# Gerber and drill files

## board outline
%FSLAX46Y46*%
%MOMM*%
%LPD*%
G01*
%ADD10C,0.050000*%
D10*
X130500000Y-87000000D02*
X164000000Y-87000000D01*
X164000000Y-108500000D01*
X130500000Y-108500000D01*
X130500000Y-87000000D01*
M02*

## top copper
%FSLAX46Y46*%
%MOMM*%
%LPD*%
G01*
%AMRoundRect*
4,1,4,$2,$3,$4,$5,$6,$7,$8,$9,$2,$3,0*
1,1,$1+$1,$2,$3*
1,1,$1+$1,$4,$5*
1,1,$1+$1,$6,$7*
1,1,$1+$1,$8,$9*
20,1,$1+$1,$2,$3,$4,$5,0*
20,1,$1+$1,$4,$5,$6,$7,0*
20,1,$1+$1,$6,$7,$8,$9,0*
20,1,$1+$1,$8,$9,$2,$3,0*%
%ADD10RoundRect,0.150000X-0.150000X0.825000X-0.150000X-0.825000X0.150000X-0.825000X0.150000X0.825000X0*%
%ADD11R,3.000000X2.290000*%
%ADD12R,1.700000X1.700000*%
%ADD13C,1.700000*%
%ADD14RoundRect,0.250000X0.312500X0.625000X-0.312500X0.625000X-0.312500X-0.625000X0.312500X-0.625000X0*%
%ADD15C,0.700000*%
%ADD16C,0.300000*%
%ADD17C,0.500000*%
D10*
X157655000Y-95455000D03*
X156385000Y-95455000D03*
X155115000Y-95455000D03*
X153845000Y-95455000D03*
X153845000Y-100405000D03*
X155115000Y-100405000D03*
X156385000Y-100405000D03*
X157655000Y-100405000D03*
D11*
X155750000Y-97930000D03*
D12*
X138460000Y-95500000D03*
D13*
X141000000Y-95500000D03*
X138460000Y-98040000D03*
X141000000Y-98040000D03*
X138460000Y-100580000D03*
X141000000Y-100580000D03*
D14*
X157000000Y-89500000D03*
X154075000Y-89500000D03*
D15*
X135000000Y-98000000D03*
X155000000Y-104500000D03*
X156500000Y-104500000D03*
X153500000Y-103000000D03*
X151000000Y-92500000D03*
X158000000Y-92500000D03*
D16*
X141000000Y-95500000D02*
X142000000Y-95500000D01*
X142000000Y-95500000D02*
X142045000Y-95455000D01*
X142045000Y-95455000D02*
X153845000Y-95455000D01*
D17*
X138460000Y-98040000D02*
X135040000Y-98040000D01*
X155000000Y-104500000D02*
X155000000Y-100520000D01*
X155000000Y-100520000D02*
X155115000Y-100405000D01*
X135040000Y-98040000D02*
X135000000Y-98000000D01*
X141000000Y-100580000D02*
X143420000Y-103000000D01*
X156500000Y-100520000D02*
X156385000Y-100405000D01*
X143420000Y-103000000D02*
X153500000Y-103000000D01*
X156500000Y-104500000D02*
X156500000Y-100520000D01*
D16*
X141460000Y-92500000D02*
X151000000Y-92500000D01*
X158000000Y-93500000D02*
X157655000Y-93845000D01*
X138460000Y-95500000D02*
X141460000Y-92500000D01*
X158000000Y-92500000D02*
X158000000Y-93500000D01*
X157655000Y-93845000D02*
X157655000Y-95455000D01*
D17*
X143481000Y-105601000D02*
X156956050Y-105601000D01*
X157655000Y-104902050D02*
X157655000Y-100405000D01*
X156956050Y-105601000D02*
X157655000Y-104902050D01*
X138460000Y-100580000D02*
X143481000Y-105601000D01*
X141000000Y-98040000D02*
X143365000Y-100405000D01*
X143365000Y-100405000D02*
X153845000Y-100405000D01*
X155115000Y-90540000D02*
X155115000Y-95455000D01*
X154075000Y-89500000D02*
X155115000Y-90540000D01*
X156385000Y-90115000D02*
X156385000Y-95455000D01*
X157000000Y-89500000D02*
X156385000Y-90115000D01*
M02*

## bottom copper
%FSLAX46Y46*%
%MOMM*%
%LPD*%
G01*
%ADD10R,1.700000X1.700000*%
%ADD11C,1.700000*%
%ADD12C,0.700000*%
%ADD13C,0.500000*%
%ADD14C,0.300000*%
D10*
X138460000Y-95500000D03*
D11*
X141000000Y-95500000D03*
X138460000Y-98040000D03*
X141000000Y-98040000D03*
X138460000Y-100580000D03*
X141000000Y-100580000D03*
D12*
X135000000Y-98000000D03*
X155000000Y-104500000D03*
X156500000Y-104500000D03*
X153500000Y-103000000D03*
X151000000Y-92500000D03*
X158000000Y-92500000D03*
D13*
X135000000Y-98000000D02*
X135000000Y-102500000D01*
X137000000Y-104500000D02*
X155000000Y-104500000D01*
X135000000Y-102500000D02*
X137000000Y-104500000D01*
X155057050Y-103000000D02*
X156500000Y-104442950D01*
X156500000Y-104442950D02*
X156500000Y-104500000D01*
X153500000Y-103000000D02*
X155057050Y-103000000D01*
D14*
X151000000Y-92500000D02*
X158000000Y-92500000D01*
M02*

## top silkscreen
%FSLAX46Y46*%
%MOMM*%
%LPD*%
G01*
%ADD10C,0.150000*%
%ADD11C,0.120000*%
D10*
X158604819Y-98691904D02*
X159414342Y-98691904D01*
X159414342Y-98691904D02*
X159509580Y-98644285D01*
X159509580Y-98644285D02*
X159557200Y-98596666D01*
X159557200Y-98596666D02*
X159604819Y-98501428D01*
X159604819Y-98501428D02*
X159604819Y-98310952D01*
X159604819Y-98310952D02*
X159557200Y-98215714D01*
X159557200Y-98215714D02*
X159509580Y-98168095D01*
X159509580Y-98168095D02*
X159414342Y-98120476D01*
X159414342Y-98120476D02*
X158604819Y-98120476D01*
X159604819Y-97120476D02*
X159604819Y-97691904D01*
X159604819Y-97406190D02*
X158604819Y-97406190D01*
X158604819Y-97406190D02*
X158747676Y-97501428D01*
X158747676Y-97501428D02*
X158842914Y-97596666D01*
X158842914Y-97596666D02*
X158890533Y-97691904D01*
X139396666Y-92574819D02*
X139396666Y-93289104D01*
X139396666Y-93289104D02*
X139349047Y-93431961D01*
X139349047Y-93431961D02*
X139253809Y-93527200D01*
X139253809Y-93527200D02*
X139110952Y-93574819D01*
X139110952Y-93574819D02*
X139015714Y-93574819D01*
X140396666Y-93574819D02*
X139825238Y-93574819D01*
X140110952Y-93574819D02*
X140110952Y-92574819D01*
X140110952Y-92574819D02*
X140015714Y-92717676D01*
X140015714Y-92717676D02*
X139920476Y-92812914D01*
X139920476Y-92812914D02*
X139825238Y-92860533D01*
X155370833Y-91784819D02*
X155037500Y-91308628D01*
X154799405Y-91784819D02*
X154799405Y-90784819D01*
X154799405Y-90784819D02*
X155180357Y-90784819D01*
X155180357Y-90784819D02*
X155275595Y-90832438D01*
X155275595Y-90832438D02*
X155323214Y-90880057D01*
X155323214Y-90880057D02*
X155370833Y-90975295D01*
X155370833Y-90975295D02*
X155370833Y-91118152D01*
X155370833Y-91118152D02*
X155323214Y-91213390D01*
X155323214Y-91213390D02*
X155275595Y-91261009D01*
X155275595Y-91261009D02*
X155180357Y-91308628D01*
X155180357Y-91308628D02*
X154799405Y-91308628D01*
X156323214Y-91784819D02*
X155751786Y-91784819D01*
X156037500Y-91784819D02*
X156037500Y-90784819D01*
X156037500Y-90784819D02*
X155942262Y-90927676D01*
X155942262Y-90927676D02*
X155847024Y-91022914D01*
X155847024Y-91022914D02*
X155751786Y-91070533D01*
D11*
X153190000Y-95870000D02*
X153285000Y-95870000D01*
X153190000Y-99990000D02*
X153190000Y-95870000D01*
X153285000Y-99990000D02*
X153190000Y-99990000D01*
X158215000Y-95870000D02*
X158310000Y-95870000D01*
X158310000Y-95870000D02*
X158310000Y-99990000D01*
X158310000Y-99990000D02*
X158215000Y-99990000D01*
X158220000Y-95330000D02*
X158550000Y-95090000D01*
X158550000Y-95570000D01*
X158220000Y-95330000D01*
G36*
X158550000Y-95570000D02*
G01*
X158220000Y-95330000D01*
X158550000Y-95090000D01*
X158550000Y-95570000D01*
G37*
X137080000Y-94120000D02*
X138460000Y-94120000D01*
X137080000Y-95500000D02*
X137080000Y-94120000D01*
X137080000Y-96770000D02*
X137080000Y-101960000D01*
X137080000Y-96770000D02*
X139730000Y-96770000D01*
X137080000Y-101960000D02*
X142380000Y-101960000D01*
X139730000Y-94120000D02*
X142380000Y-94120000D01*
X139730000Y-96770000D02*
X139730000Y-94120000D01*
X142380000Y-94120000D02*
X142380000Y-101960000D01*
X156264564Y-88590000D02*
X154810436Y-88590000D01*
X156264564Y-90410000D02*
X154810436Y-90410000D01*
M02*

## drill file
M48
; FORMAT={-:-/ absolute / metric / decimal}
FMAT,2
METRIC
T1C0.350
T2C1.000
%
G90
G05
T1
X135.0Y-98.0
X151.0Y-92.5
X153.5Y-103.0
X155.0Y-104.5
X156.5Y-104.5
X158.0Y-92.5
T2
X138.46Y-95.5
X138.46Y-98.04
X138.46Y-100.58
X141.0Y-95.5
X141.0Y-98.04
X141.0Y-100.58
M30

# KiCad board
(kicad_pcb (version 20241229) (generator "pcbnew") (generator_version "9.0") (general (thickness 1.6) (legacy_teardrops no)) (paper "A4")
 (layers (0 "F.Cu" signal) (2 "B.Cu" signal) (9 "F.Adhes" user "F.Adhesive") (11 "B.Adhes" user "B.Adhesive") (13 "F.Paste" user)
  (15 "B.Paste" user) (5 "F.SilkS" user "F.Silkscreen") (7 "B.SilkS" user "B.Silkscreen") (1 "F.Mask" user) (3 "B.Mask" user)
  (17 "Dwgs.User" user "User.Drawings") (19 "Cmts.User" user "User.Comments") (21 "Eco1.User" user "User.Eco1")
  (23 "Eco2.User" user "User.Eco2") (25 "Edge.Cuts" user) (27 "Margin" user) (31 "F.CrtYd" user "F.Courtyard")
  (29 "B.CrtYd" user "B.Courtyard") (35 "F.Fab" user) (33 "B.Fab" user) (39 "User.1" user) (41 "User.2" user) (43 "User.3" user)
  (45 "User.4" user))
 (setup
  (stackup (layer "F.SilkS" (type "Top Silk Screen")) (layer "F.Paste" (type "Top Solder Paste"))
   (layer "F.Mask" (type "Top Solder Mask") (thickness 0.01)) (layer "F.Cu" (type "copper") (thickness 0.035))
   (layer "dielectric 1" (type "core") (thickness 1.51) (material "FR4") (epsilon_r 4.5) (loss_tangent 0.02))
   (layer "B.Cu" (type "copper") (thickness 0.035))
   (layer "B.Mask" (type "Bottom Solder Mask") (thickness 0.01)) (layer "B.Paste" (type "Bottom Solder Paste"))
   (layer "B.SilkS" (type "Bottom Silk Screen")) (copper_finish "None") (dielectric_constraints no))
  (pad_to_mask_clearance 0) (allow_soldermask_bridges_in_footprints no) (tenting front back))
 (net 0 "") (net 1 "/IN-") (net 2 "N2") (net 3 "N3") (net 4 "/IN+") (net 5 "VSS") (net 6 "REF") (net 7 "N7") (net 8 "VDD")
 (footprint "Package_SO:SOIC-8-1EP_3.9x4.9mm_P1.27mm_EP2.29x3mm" (layer "F.Cu") (at 155.75 97.93 -90)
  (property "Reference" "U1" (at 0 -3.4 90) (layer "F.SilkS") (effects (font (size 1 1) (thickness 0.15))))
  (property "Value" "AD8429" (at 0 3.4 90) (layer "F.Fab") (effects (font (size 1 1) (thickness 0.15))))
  (fp_line (start -2.06 2.56) (end -2.06 2.465) (stroke (width 0.12) (type solid)) (layer "F.SilkS"))
  (fp_line (start 2.06 2.56) (end -2.06 2.56) (stroke (width 0.12) (type solid)) (layer "F.SilkS"))
  (fp_line (start 2.06 2.465) (end 2.06 2.56) (stroke (width 0.12) (type solid)) (layer "F.SilkS"))
  (fp_line (start -2.06 -2.465) (end -2.06 -2.56) (stroke (width 0.12) (type solid)) (layer "F.SilkS"))
  (fp_line (start -2.06 -2.56) (end 2.06 -2.56) (stroke (width 0.12) (type solid)) (layer "F.SilkS"))
  (fp_line (start 2.06 -2.56) (end 2.06 -2.465) (stroke (width 0.12) (type solid)) (layer "F.SilkS"))
  (fp_poly (pts (xy -2.6 -2.47) (xy -2.84 -2.8) (xy -2.36 -2.8)) (stroke (width 0.12) (type solid)) (fill yes) (layer "F.SilkS"))
  (pad "" smd roundrect (at -0.57 -0.75 270) (size 0.92 1.21) (layers "F.Paste") (roundrect_rratio 0.25))
  (pad "" smd roundrect (at -0.57 0.75 270) (size 0.92 1.21) (layers "F.Paste") (roundrect_rratio 0.25))
  (pad "" smd roundrect (at 0.57 -0.75 270) (size 0.92 1.21) (layers "F.Paste") (roundrect_rratio 0.25))
  (pad "" smd roundrect (at 0.57 0.75 270) (size 0.92 1.21) (layers "F.Paste") (roundrect_rratio 0.25))
  (pad "1" smd roundrect (at -2.475 -1.905 270) (size 1.95 0.6) (layers "F.Cu" "F.Mask" "F.Paste") (roundrect_rratio 0.25) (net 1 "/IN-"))
  (pad "2" smd roundrect (at -2.475 -0.635 270) (size 1.95 0.6) (layers "F.Cu" "F.Mask" "F.Paste") (roundrect_rratio 0.25) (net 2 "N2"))
  (pad "3" smd roundrect (at -2.475 0.635 270) (size 1.95 0.6) (layers "F.Cu" "F.Mask" "F.Paste") (roundrect_rratio 0.25) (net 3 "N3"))
  (pad "4" smd roundrect (at -2.475 1.905 270) (size 1.95 0.6) (layers "F.Cu" "F.Mask" "F.Paste") (roundrect_rratio 0.25) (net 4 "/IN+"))
  (pad "5" smd roundrect (at 2.475 1.905 270) (size 1.95 0.6) (layers "F.Cu" "F.Mask" "F.Paste") (roundrect_rratio 0.25) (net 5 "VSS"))
  (pad "6" smd roundrect (at 2.475 0.635 270) (size 1.95 0.6) (layers "F.Cu" "F.Mask" "F.Paste") (roundrect_rratio 0.25) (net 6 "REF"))
  (pad "7" smd roundrect (at 2.475 -0.635 270) (size 1.95 0.6) (layers "F.Cu" "F.Mask" "F.Paste") (roundrect_rratio 0.25) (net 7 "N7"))
  (pad "8" smd roundrect (at 2.475 -1.905 270) (size 1.95 0.6) (layers "F.Cu" "F.Mask" "F.Paste") (roundrect_rratio 0.25) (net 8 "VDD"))
  (pad "9" smd rect (at 0 0 270) (size 2.29 3) (layers "F.Cu" "F.Mask") (zone_connect 2)))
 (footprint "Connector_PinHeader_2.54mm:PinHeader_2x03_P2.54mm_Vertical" (layer "F.Cu") (at 138.46 95.5)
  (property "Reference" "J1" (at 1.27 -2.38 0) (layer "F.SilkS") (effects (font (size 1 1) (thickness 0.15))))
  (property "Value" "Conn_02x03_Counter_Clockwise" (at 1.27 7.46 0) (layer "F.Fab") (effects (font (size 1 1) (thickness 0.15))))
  (fp_line (start -1.38 -1.38) (end 0 -1.38) (stroke (width 0.12) (type solid)) (layer "F.SilkS"))
  (fp_line (start -1.38 0) (end -1.38 -1.38) (stroke (width 0.12) (type solid)) (layer "F.SilkS"))
  (fp_line (start -1.38 1.27) (end -1.38 6.46) (stroke (width 0.12) (type solid)) (layer "F.SilkS"))
  (fp_line (start -1.38 1.27) (end 1.27 1.27) (stroke (width 0.12) (type solid)) (layer "F.SilkS"))
  (fp_line (start -1.38 6.46) (end 3.92 6.46) (stroke (width 0.12) (type solid)) (layer "F.SilkS"))
  (fp_line (start 1.27 -1.38) (end 3.92 -1.38) (stroke (width 0.12) (type solid)) (layer "F.SilkS"))
  (fp_line (start 1.27 1.27) (end 1.27 -1.38) (stroke (width 0.12) (type solid)) (layer "F.SilkS"))
  (fp_line (start 3.92 -1.38) (end 3.92 6.46) (stroke (width 0.12) (type solid)) (layer "F.SilkS"))
  (pad "1" thru_hole rect (at 0 0) (size 1.7 1.7) (drill 1) (layers "*.Cu" "*.Mask") (remove_unused_layers no) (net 1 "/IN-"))
  (pad "2" thru_hole circle (at 2.54 0) (size 1.7 1.7) (drill 1) (layers "*.Cu" "*.Mask") (remove_unused_layers no) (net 4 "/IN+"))
  (pad "3" thru_hole circle (at 0 2.54) (size 1.7 1.7) (drill 1) (layers "*.Cu" "*.Mask") (remove_unused_layers no) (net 6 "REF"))
  (pad "4" thru_hole circle (at 2.54 2.54) (size 1.7 1.7) (drill 1) (layers "*.Cu" "*.Mask") (remove_unused_layers no) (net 5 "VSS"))
  (pad "5" thru_hole circle (at 0 5.08) (size 1.7 1.7) (drill 1) (layers "*.Cu" "*.Mask") (remove_unused_layers no) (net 8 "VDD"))
  (pad "6" thru_hole circle (at 2.54 5.08) (size 1.7 1.7) (drill 1) (layers "*.Cu" "*.Mask") (remove_unused_layers no) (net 7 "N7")))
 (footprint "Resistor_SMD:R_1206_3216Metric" (layer "F.Cu") (at 155.5375 89.5 180)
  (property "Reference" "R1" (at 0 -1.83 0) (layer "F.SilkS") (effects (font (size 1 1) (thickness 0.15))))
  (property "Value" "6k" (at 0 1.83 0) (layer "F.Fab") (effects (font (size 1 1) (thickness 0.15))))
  (fp_line (start -0.727064 0.91) (end 0.727064 0.91) (stroke (width 0.12) (type solid)) (layer "F.SilkS"))
  (fp_line (start -0.727064 -0.91) (end 0.727064 -0.91) (stroke (width 0.12) (type solid)) (layer "F.SilkS"))
  (pad "1" smd roundrect (at -1.4625 0 180) (size 1.125 1.75) (layers "F.Cu" "F.Mask" "F.Paste") (roundrect_rratio 0.222222) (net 2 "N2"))
  (pad "2" smd roundrect (at 1.4625 0 180) (size 1.125 1.75) (layers "F.Cu" "F.Mask" "F.Paste") (roundrect_rratio 0.222222) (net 3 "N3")))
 (gr_rect (start 130.5 87) (end 164 108.5) (stroke (width 0.05) (type default)) (fill no) (layer "Edge.Cuts"))
 (segment (start 141 95.5) (end 142 95.5) (width 0.3) (layer "F.Cu") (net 4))
 (segment (start 142 95.5) (end 142.045 95.455) (width 0.3) (layer "F.Cu") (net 4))
 (segment (start 142.045 95.455) (end 153.845 95.455) (width 0.3) (layer "F.Cu") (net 4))
 (segment (start 138.46 98.04) (end 135.04 98.04) (width 0.5) (layer "F.Cu") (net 6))
 (segment (start 155 104.5) (end 155 100.52) (width 0.5) (layer "F.Cu") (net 6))
 (segment (start 155 100.52) (end 155.115 100.405) (width 0.5) (layer "F.Cu") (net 6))
 (segment (start 135.04 98.04) (end 135 98) (width 0.5) (layer "F.Cu") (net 6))
 (via (at 135 98) (size 0.7) (drill 0.35) (layers "F.Cu" "B.Cu") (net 6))
 (via (at 155 104.5) (size 0.7) (drill 0.35) (layers "F.Cu" "B.Cu") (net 6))
 (segment (start 135 98) (end 135 102.5) (width 0.5) (layer "B.Cu") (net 6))
 (segment (start 137 104.5) (end 155 104.5) (width 0.5) (layer "B.Cu") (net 6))
 (segment (start 135 102.5) (end 137 104.5) (width 0.5) (layer "B.Cu") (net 6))
 (segment (start 141 100.58) (end 143.42 103) (width 0.5) (layer "F.Cu") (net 7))
 (segment (start 156.5 100.52) (end 156.385 100.405) (width 0.5) (layer "F.Cu") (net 7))
 (segment (start 143.42 103) (end 153.5 103) (width 0.5) (layer "F.Cu") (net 7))
 (segment (start 156.5 104.5) (end 156.5 100.52) (width 0.5) (layer "F.Cu") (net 7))
 (via (at 156.5 104.5) (size 0.7) (drill 0.35) (layers "F.Cu" "B.Cu") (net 7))
 (via (at 153.5 103) (size 0.7) (drill 0.35) (layers "F.Cu" "B.Cu") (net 7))
 (segment (start 155.05705 103) (end 156.5 104.44295) (width 0.5) (layer "B.Cu") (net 7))
 (segment (start 156.5 104.44295) (end 156.5 104.5) (width 0.5) (layer "B.Cu") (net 7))
 (segment (start 153.5 103) (end 155.05705 103) (width 0.5) (layer "B.Cu") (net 7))
 (segment (start 141.46 92.5) (end 151 92.5) (width 0.3) (layer "F.Cu") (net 1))
 (segment (start 158 93.5) (end 157.655 93.845) (width 0.3) (layer "F.Cu") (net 1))
 (segment (start 138.46 95.5) (end 141.46 92.5) (width 0.3) (layer "F.Cu") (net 1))
 (segment (start 158 92.5) (end 158 93.5) (width 0.3) (layer "F.Cu") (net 1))
 (segment (start 157.655 93.845) (end 157.655 95.455) (width 0.3) (layer "F.Cu") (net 1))
 (via (at 151 92.5) (size 0.7) (drill 0.35) (layers "F.Cu" "B.Cu") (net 1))
 (via (at 158 92.5) (size 0.7) (drill 0.35) (layers "F.Cu" "B.Cu") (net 1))
 (segment (start 151 92.5) (end 158 92.5) (width 0.3) (layer "B.Cu") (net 1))
 (segment (start 143.481 105.601) (end 156.95605 105.601) (width 0.5) (layer "F.Cu") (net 8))
 (segment (start 157.655 104.90205) (end 157.655 100.405) (width 0.5) (layer "F.Cu") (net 8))
 (segment (start 156.95605 105.601) (end 157.655 104.90205) (width 0.5) (layer "F.Cu") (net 8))
 (segment (start 138.46 100.58) (end 143.481 105.601) (width 0.5) (layer "F.Cu") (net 8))
 (segment (start 141 98.04) (end 143.365 100.405) (width 0.5) (layer "F.Cu") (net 5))
 (segment (start 143.365 100.405) (end 153.845 100.405) (width 0.5) (layer "F.Cu") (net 5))
 (segment (start 155.115 90.54) (end 155.115 95.455) (width 0.5) (layer "F.Cu") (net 3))
 (segment (start 154.075 89.5) (end 155.115 90.54) (width 0.5) (layer "F.Cu") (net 3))
 (segment (start 156.385 90.115) (end 156.385 95.455) (width 0.5) (layer "F.Cu") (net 2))
 (segment (start 157 89.5) (end 156.385 90.115) (width 0.5) (layer "F.Cu") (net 2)))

